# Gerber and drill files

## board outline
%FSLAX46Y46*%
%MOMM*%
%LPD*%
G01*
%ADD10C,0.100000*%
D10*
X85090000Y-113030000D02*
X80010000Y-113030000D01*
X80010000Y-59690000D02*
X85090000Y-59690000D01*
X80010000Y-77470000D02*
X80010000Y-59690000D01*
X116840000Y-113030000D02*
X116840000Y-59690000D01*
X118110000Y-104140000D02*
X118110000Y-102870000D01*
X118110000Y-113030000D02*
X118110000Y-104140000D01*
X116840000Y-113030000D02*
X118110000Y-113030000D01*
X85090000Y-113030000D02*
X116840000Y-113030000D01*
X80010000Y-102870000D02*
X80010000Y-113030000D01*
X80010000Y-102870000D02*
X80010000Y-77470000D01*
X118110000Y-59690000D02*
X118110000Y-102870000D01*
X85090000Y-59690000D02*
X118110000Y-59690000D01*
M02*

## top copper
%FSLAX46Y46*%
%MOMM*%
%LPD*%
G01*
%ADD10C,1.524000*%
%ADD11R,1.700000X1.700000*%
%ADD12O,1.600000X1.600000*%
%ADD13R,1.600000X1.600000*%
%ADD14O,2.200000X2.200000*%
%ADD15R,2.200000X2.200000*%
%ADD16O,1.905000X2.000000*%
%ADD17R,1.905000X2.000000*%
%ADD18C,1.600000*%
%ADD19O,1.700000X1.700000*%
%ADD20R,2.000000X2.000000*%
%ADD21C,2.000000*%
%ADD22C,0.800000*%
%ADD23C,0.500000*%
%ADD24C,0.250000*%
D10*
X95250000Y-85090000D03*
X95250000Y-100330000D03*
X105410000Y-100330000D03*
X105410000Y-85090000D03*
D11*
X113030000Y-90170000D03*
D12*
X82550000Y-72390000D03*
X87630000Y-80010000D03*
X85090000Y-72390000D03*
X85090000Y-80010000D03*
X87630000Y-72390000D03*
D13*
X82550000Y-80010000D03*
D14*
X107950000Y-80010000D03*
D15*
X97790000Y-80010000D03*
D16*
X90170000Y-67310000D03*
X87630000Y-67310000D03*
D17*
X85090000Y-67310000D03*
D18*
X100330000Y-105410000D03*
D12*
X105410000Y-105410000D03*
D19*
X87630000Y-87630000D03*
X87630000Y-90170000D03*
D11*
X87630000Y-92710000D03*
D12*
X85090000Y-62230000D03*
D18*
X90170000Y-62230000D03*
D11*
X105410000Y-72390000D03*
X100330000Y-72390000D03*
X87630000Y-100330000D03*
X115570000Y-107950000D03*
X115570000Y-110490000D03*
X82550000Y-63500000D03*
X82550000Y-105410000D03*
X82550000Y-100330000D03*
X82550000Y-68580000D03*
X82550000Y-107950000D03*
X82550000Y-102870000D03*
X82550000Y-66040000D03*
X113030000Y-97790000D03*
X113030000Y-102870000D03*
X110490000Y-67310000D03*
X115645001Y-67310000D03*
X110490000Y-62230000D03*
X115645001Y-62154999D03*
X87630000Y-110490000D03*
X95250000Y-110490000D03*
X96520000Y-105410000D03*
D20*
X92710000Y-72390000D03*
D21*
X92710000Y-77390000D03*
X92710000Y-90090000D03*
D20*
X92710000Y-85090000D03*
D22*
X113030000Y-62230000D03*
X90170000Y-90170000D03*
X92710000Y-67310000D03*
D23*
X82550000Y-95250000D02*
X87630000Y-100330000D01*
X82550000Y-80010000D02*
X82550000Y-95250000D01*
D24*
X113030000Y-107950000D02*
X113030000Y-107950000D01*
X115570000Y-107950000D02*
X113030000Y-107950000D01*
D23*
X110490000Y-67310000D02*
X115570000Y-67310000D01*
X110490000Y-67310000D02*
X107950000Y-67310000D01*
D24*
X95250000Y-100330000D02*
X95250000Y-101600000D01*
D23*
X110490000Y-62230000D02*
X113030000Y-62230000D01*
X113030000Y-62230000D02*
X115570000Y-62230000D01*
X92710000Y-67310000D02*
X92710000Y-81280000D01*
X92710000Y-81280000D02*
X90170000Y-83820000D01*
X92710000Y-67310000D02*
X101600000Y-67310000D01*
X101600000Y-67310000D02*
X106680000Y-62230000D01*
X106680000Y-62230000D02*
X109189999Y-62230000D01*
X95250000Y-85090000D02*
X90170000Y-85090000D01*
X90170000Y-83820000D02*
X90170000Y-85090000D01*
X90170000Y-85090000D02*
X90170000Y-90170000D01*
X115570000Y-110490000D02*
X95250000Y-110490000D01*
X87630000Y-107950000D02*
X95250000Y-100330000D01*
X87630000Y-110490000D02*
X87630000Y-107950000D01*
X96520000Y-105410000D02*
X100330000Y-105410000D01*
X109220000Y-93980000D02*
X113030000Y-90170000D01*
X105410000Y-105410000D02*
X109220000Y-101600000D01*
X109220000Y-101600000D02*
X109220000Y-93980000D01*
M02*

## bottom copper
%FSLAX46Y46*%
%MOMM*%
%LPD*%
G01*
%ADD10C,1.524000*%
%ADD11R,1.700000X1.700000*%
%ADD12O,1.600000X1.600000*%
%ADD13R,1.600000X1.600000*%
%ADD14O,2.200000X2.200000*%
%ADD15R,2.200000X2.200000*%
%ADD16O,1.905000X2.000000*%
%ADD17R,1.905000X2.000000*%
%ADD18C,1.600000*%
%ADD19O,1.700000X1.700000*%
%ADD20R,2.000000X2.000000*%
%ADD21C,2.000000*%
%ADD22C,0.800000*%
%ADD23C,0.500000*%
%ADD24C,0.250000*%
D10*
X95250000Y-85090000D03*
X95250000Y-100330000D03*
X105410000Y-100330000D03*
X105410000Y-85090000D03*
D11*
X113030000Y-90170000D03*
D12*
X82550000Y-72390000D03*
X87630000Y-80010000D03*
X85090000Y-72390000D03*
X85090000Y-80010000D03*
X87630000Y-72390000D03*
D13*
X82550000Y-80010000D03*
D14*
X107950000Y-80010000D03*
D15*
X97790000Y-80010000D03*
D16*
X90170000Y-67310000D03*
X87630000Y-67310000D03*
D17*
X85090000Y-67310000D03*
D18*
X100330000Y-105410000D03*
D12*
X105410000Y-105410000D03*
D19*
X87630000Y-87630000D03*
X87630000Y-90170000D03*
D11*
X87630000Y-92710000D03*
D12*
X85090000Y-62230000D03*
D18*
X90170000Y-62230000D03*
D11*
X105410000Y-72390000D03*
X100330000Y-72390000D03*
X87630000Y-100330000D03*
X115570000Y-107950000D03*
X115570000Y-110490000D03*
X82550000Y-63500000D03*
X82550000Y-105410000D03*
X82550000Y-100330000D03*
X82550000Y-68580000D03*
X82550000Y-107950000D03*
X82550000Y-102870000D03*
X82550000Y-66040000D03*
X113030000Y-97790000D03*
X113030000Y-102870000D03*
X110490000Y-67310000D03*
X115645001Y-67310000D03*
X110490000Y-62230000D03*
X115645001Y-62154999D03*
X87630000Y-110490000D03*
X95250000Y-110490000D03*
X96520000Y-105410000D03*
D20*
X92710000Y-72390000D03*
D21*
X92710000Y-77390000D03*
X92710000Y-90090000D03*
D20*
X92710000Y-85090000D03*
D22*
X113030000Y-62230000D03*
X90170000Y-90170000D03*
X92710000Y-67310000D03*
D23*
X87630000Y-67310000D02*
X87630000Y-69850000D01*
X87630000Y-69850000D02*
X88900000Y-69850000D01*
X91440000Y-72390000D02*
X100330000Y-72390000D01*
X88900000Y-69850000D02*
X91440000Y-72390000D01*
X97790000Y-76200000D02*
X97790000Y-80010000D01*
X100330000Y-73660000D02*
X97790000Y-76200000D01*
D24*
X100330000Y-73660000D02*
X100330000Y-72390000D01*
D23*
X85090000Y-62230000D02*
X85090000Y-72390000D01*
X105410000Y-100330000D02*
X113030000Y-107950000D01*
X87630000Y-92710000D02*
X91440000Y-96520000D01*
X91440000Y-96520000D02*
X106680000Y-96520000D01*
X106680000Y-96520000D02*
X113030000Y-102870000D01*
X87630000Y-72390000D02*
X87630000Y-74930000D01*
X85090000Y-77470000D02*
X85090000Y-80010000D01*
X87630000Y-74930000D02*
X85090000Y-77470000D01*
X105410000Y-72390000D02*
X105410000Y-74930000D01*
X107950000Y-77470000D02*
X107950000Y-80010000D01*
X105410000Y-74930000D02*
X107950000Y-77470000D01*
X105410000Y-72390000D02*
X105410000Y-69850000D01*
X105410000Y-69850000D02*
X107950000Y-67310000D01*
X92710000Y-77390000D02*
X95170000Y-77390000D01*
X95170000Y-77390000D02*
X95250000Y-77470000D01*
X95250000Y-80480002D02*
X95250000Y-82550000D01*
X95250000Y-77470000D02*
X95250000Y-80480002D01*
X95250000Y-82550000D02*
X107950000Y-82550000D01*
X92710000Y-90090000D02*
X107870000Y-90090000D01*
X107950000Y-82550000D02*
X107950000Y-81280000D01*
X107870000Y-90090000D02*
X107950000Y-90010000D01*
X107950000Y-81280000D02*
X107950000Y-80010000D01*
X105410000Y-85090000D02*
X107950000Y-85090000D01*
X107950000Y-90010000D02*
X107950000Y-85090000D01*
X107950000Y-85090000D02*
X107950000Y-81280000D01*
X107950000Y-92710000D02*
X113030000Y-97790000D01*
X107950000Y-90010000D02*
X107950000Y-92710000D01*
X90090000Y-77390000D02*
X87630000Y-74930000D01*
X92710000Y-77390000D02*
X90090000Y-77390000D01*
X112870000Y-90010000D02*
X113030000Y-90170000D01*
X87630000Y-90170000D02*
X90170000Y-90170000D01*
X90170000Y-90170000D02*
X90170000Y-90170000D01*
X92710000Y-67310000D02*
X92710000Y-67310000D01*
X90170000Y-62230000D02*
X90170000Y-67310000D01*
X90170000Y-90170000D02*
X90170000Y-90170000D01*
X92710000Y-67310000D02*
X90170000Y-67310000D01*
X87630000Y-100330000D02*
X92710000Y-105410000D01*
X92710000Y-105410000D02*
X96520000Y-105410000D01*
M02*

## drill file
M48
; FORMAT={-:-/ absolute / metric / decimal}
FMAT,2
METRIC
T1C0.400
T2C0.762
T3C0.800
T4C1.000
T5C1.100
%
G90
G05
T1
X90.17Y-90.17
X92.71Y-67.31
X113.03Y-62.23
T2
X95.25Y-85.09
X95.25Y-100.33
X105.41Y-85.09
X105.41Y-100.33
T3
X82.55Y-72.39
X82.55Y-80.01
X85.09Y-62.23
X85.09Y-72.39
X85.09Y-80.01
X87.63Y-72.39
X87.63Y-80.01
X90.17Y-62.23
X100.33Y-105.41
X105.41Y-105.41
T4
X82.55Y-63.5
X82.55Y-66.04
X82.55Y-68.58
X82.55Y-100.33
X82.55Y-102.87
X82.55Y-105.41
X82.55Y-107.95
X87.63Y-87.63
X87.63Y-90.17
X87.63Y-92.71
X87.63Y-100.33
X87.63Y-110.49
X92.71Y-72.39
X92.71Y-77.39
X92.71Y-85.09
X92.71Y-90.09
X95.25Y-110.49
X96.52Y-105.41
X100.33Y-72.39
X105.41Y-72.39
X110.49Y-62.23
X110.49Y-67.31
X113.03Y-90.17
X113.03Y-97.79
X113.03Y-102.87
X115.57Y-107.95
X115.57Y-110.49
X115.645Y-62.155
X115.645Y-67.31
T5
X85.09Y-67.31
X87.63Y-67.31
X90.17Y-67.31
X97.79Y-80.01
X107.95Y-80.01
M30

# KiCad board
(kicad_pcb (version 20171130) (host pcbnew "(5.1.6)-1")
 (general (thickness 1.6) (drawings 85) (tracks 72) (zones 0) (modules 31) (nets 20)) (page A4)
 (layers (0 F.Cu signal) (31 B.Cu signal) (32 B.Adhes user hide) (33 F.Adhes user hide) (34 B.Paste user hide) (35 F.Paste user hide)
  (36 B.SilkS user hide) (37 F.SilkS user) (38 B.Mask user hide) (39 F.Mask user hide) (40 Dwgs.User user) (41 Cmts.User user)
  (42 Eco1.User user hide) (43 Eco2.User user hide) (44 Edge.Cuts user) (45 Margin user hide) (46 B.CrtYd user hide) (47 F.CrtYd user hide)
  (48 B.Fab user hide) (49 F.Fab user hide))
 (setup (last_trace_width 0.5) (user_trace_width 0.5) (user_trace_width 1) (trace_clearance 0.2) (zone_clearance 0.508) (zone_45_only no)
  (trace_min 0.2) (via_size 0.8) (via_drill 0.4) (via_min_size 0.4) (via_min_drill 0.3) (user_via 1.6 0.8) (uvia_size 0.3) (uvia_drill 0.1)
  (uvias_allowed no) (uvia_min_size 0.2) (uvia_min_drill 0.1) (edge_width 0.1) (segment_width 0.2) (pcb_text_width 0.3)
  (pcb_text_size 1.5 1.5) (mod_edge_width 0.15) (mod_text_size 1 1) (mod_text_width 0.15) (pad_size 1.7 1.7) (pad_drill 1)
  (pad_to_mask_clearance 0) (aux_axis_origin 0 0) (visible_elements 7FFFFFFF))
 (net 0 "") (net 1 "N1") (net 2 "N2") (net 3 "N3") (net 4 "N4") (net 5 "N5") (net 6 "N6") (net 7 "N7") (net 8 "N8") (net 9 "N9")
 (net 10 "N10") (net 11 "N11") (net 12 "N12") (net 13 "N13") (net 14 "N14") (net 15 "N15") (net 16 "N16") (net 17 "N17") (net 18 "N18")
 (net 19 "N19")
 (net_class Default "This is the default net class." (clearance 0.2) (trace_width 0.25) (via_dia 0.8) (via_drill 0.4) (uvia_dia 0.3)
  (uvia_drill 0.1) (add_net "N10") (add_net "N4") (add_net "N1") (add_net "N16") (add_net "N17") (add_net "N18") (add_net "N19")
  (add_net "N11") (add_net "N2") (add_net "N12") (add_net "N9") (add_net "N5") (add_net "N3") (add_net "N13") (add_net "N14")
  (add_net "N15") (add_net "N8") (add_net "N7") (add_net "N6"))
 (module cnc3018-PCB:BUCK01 (layer F.Cu) (at 105.41 90.17 270)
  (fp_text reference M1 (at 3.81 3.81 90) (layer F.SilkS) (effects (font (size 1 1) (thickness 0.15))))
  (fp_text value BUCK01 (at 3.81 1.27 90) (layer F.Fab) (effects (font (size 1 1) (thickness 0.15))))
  (pad 4 thru_hole circle (at -5.08 10.16 270) (size 1.524 1.524) (drill 0.762) (layers *.Cu *.Mask) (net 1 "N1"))
  (pad 3 thru_hole circle (at 10.16 10.16 270) (size 1.524 1.524) (drill 0.762) (layers *.Cu *.Mask) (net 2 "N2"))
  (pad 2 thru_hole circle (at 10.16 0 270) (size 1.524 1.524) (drill 0.762) (layers *.Cu *.Mask) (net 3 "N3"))
  (pad 1 thru_hole circle (at -5.08 0 270) (size 1.524 1.524) (drill 0.762) (layers *.Cu *.Mask) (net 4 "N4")))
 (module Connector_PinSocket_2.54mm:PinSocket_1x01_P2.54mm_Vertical (layer F.Cu) (at 113.03 90.17)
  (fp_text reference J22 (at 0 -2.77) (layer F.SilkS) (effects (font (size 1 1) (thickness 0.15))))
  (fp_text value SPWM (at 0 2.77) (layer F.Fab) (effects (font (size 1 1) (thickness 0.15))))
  (pad 1 thru_hole rect (at 0 0) (size 1.7 1.7) (drill 1) (layers *.Cu *.Mask) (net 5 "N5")))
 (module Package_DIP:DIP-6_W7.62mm (layer F.Cu) (at 82.55 80.01 90)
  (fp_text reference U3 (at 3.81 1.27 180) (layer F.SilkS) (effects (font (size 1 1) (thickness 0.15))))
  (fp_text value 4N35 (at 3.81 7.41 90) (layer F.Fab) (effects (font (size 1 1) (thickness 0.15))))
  (pad 6 thru_hole oval (at 7.62 0 90) (size 1.6 1.6) (drill 0.8) (layers *.Cu *.Mask) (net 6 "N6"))
  (pad 3 thru_hole oval (at 0 5.08 90) (size 1.6 1.6) (drill 0.8) (layers *.Cu *.Mask) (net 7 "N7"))
  (pad 5 thru_hole oval (at 7.62 2.54 90) (size 1.6 1.6) (drill 0.8) (layers *.Cu *.Mask) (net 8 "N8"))
  (pad 2 thru_hole oval (at 0 2.54 90) (size 1.6 1.6) (drill 0.8) (layers *.Cu *.Mask) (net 4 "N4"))
  (pad 4 thru_hole oval (at 7.62 5.08 90) (size 1.6 1.6) (drill 0.8) (layers *.Cu *.Mask) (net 4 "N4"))
  (pad 1 thru_hole rect (at 0 0 90) (size 1.6 1.6) (drill 0.8) (layers *.Cu *.Mask) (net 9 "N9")))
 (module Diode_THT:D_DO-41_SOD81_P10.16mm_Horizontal (layer F.Cu) (at 97.79 80.01)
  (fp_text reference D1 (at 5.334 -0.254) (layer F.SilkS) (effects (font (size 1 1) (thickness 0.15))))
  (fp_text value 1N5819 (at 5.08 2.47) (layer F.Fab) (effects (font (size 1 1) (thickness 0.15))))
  (pad 2 thru_hole oval (at 10.16 0) (size 2.2 2.2) (drill 1.1) (layers *.Cu *.Mask) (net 4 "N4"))
  (pad 1 thru_hole rect (at 0 0) (size 2.2 2.2) (drill 1.1) (layers *.Cu *.Mask) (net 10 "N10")))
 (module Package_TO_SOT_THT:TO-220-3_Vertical (layer F.Cu) (at 85.09 67.31)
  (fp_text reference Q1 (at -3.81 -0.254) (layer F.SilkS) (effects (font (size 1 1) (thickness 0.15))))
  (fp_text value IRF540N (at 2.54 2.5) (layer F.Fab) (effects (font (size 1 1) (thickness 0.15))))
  (pad 3 thru_hole oval (at 5.08 0) (size 1.905 2) (drill 1.1) (layers *.Cu *.Mask) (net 1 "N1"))
  (pad 2 thru_hole oval (at 2.54 0) (size 1.905 2) (drill 1.1) (layers *.Cu *.Mask) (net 10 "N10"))
  (pad 1 thru_hole rect (at 0 0) (size 1.905 2) (drill 1.1) (layers *.Cu *.Mask) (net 8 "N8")))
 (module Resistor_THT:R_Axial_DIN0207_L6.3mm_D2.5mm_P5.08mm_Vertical (layer F.Cu) (at 100.33 105.41)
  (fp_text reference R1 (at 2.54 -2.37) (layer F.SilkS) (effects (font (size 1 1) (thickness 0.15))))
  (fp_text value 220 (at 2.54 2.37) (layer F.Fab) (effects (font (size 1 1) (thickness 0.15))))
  (pad 1 thru_hole circle (at 0 0) (size 1.6 1.6) (drill 0.8) (layers *.Cu *.Mask) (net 9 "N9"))
  (pad 2 thru_hole oval (at 5.08 0) (size 1.6 1.6) (drill 0.8) (layers *.Cu *.Mask) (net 5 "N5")))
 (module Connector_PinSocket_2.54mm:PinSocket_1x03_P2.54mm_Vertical (layer F.Cu) (at 87.63 92.71 180)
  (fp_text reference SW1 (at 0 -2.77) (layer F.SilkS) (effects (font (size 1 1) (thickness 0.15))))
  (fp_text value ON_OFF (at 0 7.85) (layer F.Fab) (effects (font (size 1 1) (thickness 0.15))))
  (pad 3 thru_hole oval (at 0 5.08 180) (size 1.7 1.7) (drill 1) (layers *.Cu *.Mask))
  (pad 2 thru_hole oval (at 0 2.54 180) (size 1.7 1.7) (drill 1) (layers *.Cu *.Mask) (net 1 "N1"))
  (pad 1 thru_hole rect (at 0 0 180) (size 1.7 1.7) (drill 1) (layers *.Cu *.Mask) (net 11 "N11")))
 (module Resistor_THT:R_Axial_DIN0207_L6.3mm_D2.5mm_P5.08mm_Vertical (layer F.Cu) (at 90.17 62.23 180)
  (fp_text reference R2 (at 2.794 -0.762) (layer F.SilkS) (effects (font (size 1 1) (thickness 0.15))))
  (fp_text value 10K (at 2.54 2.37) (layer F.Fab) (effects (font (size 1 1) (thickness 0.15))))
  (pad 2 thru_hole oval (at 5.08 0 180) (size 1.6 1.6) (drill 0.8) (layers *.Cu *.Mask) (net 8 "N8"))
  (pad 1 thru_hole circle (at 0 0 180) (size 1.6 1.6) (drill 0.8) (layers *.Cu *.Mask) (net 1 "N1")))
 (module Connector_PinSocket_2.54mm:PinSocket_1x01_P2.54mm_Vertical (layer F.Cu) (at 105.41 72.39)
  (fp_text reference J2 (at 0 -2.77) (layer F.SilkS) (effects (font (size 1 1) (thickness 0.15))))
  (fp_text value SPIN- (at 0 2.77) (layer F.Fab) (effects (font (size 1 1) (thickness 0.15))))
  (pad 1 thru_hole rect (at 0 0) (size 1.7 1.7) (drill 1) (layers *.Cu *.Mask) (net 4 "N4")))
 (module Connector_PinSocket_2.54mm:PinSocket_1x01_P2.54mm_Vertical (layer F.Cu) (at 100.33 72.39)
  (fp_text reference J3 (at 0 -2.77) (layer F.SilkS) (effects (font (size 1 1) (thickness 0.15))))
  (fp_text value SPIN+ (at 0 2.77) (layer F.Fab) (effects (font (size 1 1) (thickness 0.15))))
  (pad 1 thru_hole rect (at 0 0) (size 1.7 1.7) (drill 1) (layers *.Cu *.Mask) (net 10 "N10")))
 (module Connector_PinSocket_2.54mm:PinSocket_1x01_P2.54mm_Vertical (layer F.Cu) (at 87.63 100.33)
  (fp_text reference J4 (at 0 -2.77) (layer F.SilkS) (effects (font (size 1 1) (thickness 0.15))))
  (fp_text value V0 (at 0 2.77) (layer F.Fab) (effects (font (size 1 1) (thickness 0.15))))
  (pad 1 thru_hole rect (at 0 0) (size 1.7 1.7) (drill 1) (layers *.Cu *.Mask) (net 9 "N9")))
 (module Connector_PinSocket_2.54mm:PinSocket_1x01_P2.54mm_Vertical (layer F.Cu) (at 115.57 107.95)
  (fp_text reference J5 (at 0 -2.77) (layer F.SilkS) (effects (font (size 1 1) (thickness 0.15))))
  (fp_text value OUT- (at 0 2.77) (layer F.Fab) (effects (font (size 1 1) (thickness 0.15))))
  (pad 1 thru_hole rect (at 0 0) (size 1.7 1.7) (drill 1) (layers *.Cu *.Mask) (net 3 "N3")))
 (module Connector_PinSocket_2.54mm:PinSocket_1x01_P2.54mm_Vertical (layer F.Cu) (at 115.57 110.49)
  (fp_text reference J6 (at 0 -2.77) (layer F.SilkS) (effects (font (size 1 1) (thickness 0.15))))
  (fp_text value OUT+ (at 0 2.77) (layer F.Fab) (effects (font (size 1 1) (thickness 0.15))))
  (pad 1 thru_hole rect (at 0 0) (size 1.7 1.7) (drill 1) (layers *.Cu *.Mask) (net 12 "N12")))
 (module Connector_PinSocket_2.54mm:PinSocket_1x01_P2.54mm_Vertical (layer F.Cu) (at 82.55 63.5)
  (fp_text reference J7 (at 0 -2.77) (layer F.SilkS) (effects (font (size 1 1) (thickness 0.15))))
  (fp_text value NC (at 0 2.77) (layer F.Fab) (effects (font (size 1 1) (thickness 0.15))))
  (pad 1 thru_hole rect (at 0 0) (size 1.7 1.7) (drill 1) (layers *.Cu *.Mask) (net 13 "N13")))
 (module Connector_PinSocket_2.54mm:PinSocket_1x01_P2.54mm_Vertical (layer F.Cu) (at 82.55 105.41)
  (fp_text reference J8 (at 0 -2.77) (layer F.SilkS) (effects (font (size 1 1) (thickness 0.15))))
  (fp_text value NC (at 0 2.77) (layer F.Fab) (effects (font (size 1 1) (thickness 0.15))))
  (pad 1 thru_hole rect (at 0 0) (size 1.7 1.7) (drill 1) (layers *.Cu *.Mask) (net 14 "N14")))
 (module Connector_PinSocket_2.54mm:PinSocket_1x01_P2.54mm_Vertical (layer F.Cu) (at 82.55 100.33)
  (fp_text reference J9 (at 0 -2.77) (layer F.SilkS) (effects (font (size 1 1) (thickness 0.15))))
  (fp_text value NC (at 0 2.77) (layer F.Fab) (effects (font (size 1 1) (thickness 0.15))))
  (pad 1 thru_hole rect (at 0 0) (size 1.7 1.7) (drill 1) (layers *.Cu *.Mask) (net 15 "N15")))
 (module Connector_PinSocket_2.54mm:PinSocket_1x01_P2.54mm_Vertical (layer F.Cu) (at 82.55 68.58)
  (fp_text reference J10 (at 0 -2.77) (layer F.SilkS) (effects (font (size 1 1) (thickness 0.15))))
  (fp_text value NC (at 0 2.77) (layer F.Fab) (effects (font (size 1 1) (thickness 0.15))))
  (pad 1 thru_hole rect (at 0 0) (size 1.7 1.7) (drill 1) (layers *.Cu *.Mask) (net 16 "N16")))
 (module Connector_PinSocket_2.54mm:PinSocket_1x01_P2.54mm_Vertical (layer F.Cu) (at 82.55 107.95)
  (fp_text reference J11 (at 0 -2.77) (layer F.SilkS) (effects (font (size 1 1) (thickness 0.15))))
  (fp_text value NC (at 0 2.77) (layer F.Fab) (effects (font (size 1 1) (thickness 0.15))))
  (pad 1 thru_hole rect (at 0 0) (size 1.7 1.7) (drill 1) (layers *.Cu *.Mask) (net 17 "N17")))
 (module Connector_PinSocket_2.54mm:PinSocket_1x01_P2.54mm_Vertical (layer F.Cu) (at 82.55 102.87)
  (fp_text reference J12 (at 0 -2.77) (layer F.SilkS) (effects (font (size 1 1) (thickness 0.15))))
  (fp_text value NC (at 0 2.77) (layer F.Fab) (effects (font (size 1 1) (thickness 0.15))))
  (pad 1 thru_hole rect (at 0 0) (size 1.7 1.7) (drill 1) (layers *.Cu *.Mask) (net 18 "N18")))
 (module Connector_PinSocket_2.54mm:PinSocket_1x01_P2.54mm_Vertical (layer F.Cu) (at 82.55 66.04)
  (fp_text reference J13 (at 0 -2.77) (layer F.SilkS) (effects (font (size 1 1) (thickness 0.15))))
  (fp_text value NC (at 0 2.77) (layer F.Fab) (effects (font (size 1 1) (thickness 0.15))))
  (pad 1 thru_hole rect (at 0 0) (size 1.7 1.7) (drill 1) (layers *.Cu *.Mask) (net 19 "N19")))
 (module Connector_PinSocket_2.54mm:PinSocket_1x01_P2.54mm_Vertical (layer F.Cu) (at 113.03 97.79 270)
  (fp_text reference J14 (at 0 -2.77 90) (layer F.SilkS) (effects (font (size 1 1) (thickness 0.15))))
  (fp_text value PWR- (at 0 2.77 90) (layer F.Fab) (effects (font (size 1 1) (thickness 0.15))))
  (pad 1 thru_hole rect (at 0 0 270) (size 1.7 1.7) (drill 1) (layers *.Cu *.Mask) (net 4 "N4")))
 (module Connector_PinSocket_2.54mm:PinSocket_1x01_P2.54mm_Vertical (layer F.Cu) (at 113.03 102.87 270)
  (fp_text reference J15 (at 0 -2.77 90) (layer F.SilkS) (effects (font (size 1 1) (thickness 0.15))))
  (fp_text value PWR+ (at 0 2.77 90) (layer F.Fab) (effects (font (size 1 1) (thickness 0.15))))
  (pad 1 thru_hole rect (at 0 0 270) (size 1.7 1.7) (drill 1) (layers *.Cu *.Mask) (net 11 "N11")))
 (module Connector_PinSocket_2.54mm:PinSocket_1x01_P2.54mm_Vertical (layer F.Cu) (at 110.49 67.31 90)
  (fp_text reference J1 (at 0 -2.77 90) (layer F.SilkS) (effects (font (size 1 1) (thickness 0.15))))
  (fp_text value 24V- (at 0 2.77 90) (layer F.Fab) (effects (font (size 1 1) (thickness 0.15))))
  (pad 1 thru_hole rect (at 0 0 90) (size 1.7 1.7) (drill 1) (layers *.Cu *.Mask) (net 4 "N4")))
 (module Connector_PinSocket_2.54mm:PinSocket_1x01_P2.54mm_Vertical (layer F.Cu) (at 115.645001 67.31 90)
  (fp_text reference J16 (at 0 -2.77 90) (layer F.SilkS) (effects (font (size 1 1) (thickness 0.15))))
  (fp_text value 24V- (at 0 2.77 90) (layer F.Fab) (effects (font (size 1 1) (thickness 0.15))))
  (pad 1 thru_hole rect (at 0 0 90) (size 1.7 1.7) (drill 1) (layers *.Cu *.Mask) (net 4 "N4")))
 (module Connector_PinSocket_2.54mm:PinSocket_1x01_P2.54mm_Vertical (layer F.Cu) (at 110.49 62.23 90)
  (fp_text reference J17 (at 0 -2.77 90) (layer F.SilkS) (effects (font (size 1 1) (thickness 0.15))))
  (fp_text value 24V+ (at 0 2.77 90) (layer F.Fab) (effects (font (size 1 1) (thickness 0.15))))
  (pad 1 thru_hole rect (at 0 0 90) (size 1.7 1.7) (drill 1) (layers *.Cu *.Mask) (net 1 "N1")))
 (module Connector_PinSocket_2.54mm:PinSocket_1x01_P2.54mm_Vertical (layer F.Cu) (at 115.645001 62.154999 90)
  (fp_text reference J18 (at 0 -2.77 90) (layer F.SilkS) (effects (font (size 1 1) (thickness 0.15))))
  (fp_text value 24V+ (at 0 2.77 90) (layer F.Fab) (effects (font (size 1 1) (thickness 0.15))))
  (pad 1 thru_hole rect (at 0 0 90) (size 1.7 1.7) (drill 1) (layers *.Cu *.Mask) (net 1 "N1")))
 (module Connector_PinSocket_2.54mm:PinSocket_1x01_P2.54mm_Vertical (layer F.Cu) (at 87.63 110.49)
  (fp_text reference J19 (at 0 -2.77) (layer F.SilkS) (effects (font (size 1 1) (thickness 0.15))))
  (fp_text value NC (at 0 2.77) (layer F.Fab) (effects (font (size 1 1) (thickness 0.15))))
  (pad 1 thru_hole rect (at 0 0) (size 1.7 1.7) (drill 1) (layers *.Cu *.Mask) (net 2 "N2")))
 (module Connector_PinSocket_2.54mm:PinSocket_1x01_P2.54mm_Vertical (layer F.Cu) (at 95.25 110.49)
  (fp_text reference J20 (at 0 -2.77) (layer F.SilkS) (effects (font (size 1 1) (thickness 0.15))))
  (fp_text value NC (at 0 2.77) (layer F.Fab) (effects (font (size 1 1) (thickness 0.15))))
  (pad 1 thru_hole rect (at 0 0) (size 1.7 1.7) (drill 1) (layers *.Cu *.Mask) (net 12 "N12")))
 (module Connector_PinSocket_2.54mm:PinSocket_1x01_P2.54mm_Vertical (layer F.Cu) (at 96.52 105.41)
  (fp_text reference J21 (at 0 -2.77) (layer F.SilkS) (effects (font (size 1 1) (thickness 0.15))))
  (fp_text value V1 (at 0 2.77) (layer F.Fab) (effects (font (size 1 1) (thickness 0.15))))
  (pad 1 thru_hole rect (at 0 0) (size 1.7 1.7) (drill 1) (layers *.Cu *.Mask) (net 9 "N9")))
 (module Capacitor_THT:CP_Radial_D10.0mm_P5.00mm (layer F.Cu) (at 92.71 72.39 270)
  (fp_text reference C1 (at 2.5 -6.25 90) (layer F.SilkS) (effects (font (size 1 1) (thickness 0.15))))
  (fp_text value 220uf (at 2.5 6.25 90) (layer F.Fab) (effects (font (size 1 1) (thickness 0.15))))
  (pad 1 thru_hole rect (at 0 0 270) (size 2 2) (drill 1) (layers *.Cu *.Mask) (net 10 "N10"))
  (pad 2 thru_hole circle (at 5 0 270) (size 2 2) (drill 1) (layers *.Cu *.Mask) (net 4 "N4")))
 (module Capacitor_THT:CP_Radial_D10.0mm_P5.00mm (layer F.Cu) (at 92.71 85.09 270)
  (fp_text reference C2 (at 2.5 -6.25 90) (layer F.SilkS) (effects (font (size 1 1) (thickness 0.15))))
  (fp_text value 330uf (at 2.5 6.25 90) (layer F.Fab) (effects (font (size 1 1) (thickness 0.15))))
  (pad 2 thru_hole circle (at 5 0 270) (size 2 2) (drill 1) (layers *.Cu *.Mask) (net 4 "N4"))
  (pad 1 thru_hole rect (at 0 0 270) (size 2 2) (drill 1) (layers *.Cu *.Mask) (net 1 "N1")))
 (gr_line (start 85.09 113.03) (end 80.01 113.03) (layer Edge.Cuts) (width 0.1))
 (gr_line (start 80.01 59.69) (end 85.09 59.69) (layer Edge.Cuts) (width 0.1))
 (gr_line (start 80.01 77.47) (end 80.01 59.69) (layer Edge.Cuts) (width 0.1))
 (gr_line (start 116.84 113.03) (end 116.84 59.69) (layer Edge.Cuts) (width 0.1))
 (gr_line (start 118.11 104.14) (end 118.11 102.87) (layer Edge.Cuts) (width 0.1))
 (gr_line (start 118.11 113.03) (end 118.11 104.14) (layer Edge.Cuts) (width 0.1))
 (gr_line (start 116.84 113.03) (end 118.11 113.03) (layer Edge.Cuts) (width 0.1))
 (gr_line (start 85.09 113.03) (end 116.84 113.03) (layer Edge.Cuts) (width 0.1))
 (gr_line (start 80.01 102.87) (end 80.01 113.03) (layer Edge.Cuts) (width 0.1))
 (gr_line (start 80.01 102.87) (end 80.01 77.47) (layer Edge.Cuts) (width 0.1))
 (gr_line (start 118.11 59.69) (end 118.11 102.87) (layer Edge.Cuts) (width 0.1))
 (gr_line (start 85.09 59.69) (end 118.11 59.69) (layer Edge.Cuts) (width 0.1))
 (segment (start 87.63 67.31) (end 87.63 69.85) (width 0.5) (layer B.Cu) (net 10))
 (segment (start 87.63 69.85) (end 88.9 69.85) (width 0.5) (layer B.Cu) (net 10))
 (segment (start 91.44 72.39) (end 100.33 72.39) (width 0.5) (layer B.Cu) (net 10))
 (segment (start 88.9 69.85) (end 91.44 72.39) (width 0.5) (layer B.Cu) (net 10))
 (segment (start 97.79 76.2) (end 97.79 80.01) (width 0.5) (layer B.Cu) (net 10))
 (segment (start 100.33 73.66) (end 97.79 76.2) (width 0.5) (layer B.Cu) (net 10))
 (segment (start 100.33 73.66) (end 100.33 72.39) (width 0.25) (layer B.Cu) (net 10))
 (segment (start 85.09 62.23) (end 85.09 72.39) (width 0.5) (layer B.Cu) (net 8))
 (segment (start 82.55 95.25) (end 87.63 100.33) (width 0.5) (layer F.Cu) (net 9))
 (segment (start 82.55 80.01) (end 82.55 95.25) (width 0.5) (layer F.Cu) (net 9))
 (segment (start 113.03 107.95) (end 113.03 107.95) (width 0.25) (layer F.Cu) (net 3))
 (segment (start 115.57 107.95) (end 113.03 107.95) (width 0.25) (layer F.Cu) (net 3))
 (segment (start 105.41 100.33) (end 113.03 107.95) (width 0.5) (layer B.Cu) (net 3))
 (segment (start 87.63 92.71) (end 91.44 96.52) (width 0.5) (layer B.Cu) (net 11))
 (segment (start 91.44 96.52) (end 106.68 96.52) (width 0.5) (layer B.Cu) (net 11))
 (segment (start 106.68 96.52) (end 113.03 102.87) (width 0.5) (layer B.Cu) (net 11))
 (segment (start 110.49 67.31) (end 115.57 67.31) (width 0.5) (layer F.Cu) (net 4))
 (segment (start 110.49 67.31) (end 107.95 67.31) (width 0.5) (layer F.Cu) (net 4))
 (segment (start 87.63 72.39) (end 87.63 74.93) (width 0.5) (layer B.Cu) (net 4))
 (segment (start 85.09 77.47) (end 85.09 80.01) (width 0.5) (layer B.Cu) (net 4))
 (segment (start 87.63 74.93) (end 85.09 77.47) (width 0.5) (layer B.Cu) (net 4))
 (segment (start 105.41 72.39) (end 105.41 74.93) (width 0.5) (layer B.Cu) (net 4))
 (segment (start 107.95 77.47) (end 107.95 80.01) (width 0.5) (layer B.Cu) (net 4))
 (segment (start 105.41 74.93) (end 107.95 77.47) (width 0.5) (layer B.Cu) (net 4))
 (segment (start 105.41 72.39) (end 105.41 69.85) (width 0.5) (layer B.Cu) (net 4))
 (segment (start 105.41 69.85) (end 107.95 67.31) (width 0.5) (layer B.Cu) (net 4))
 (segment (start 95.25 100.33) (end 95.25 101.6) (width 0.25) (layer F.Cu) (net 2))
 (segment (start 92.71 77.39) (end 95.17 77.39) (width 0.5) (layer B.Cu) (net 4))
 (segment (start 95.17 77.39) (end 95.25 77.47) (width 0.5) (layer B.Cu) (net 4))
 (segment (start 95.25 80.480002) (end 95.25 82.55) (width 0.5) (layer B.Cu) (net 4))
 (segment (start 95.25 77.47) (end 95.25 80.480002) (width 0.5) (layer B.Cu) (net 4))
 (segment (start 95.25 82.55) (end 107.95 82.55) (width 0.5) (layer B.Cu) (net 4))
 (segment (start 92.71 90.09) (end 107.87 90.09) (width 0.5) (layer B.Cu) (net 4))
 (segment (start 107.95 82.55) (end 107.95 81.28) (width 0.5) (layer B.Cu) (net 4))
 (segment (start 107.87 90.09) (end 107.95 90.01) (width 0.5) (layer B.Cu) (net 4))
 (segment (start 107.95 81.28) (end 107.95 80.01) (width 0.5) (layer B.Cu) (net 4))
 (segment (start 105.41 85.09) (end 107.95 85.09) (width 0.5) (layer B.Cu) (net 4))
 (segment (start 107.95 90.01) (end 107.95 85.09) (width 0.5) (layer B.Cu) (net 4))
 (segment (start 107.95 85.09) (end 107.95 81.28) (width 0.5) (layer B.Cu) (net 4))
 (segment (start 107.95 92.71) (end 113.03 97.79) (width 0.5) (layer B.Cu) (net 4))
 (segment (start 107.95 90.01) (end 107.95 92.71) (width 0.5) (layer B.Cu) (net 4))
 (segment (start 90.09 77.39) (end 87.63 74.93) (width 0.5) (layer B.Cu) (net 4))
 (segment (start 92.71 77.39) (end 90.09 77.39) (width 0.5) (layer B.Cu) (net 4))
 (segment (start 112.87 90.01) (end 113.03 90.17) (width 0.5) (layer B.Cu) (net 5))
 (segment (start 110.49 62.23) (end 113.03 62.23) (width 0.5) (layer F.Cu) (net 1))
 (segment (start 113.03 62.23) (end 115.57 62.23) (width 0.5) (layer F.Cu) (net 1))
 (via (at 113.03 62.23) (size 0.8) (drill 0.4) (layers F.Cu B.Cu) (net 1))
 (segment (start 87.63 90.17) (end 90.17 90.17) (width 0.5) (layer B.Cu) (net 1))
 (segment (start 90.17 90.17) (end 90.17 90.17) (width 0.5) (layer B.Cu) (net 1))
 (segment (start 92.71 67.31) (end 92.71 67.31) (width 0.5) (layer B.Cu) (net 1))
 (segment (start 90.17 62.23) (end 90.17 67.31) (width 0.5) (layer B.Cu) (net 1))
 (segment (start 90.17 90.17) (end 90.17 90.17) (width 0.5) (layer B.Cu) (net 1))
 (via (at 90.17 90.17) (size 0.8) (drill 0.4) (layers F.Cu B.Cu) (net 1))
 (segment (start 92.71 67.31) (end 90.17 67.31) (width 0.5) (layer B.Cu) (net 1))
 (via (at 92.71 67.31) (size 0.8) (drill 0.4) (layers F.Cu B.Cu) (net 1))
 (segment (start 92.71 67.31) (end 92.71 81.28) (width 0.5) (layer F.Cu) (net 1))
 (segment (start 92.71 81.28) (end 90.17 83.82) (width 0.5) (layer F.Cu) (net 1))
 (segment (start 92.71 67.31) (end 101.6 67.31) (width 0.5) (layer F.Cu) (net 1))
 (segment (start 101.6 67.31) (end 106.68 62.23) (width 0.5) (layer F.Cu) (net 1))
 (segment (start 106.68 62.23) (end 109.189999 62.23) (width 0.5) (layer F.Cu) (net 1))
 (segment (start 95.25 85.09) (end 90.17 85.09) (width 0.5) (layer F.Cu) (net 1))
 (segment (start 90.17 83.82) (end 90.17 85.09) (width 0.5) (layer F.Cu) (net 1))
 (segment (start 90.17 85.09) (end 90.17 90.17) (width 0.5) (layer F.Cu) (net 1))
 (segment (start 115.57 110.49) (end 95.25 110.49) (width 0.5) (layer F.Cu) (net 12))
 (segment (start 87.63 107.95) (end 95.25 100.33) (width 0.5) (layer F.Cu) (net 2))
 (segment (start 87.63 110.49) (end 87.63 107.95) (width 0.5) (layer F.Cu) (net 2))
 (segment (start 87.63 100.33) (end 92.71 105.41) (width 0.5) (layer B.Cu) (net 9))
 (segment (start 92.71 105.41) (end 96.52 105.41) (width 0.5) (layer B.Cu) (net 9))
 (segment (start 96.52 105.41) (end 100.33 105.41) (width 0.5) (layer F.Cu) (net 9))
 (segment (start 109.22 93.98) (end 113.03 90.17) (width 0.5) (layer F.Cu) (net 5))
 (segment (start 105.41 105.41) (end 109.22 101.6) (width 0.5) (layer F.Cu) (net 5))
 (segment (start 109.22 101.6) (end 109.22 93.98) (width 0.5) (layer F.Cu) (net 5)))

